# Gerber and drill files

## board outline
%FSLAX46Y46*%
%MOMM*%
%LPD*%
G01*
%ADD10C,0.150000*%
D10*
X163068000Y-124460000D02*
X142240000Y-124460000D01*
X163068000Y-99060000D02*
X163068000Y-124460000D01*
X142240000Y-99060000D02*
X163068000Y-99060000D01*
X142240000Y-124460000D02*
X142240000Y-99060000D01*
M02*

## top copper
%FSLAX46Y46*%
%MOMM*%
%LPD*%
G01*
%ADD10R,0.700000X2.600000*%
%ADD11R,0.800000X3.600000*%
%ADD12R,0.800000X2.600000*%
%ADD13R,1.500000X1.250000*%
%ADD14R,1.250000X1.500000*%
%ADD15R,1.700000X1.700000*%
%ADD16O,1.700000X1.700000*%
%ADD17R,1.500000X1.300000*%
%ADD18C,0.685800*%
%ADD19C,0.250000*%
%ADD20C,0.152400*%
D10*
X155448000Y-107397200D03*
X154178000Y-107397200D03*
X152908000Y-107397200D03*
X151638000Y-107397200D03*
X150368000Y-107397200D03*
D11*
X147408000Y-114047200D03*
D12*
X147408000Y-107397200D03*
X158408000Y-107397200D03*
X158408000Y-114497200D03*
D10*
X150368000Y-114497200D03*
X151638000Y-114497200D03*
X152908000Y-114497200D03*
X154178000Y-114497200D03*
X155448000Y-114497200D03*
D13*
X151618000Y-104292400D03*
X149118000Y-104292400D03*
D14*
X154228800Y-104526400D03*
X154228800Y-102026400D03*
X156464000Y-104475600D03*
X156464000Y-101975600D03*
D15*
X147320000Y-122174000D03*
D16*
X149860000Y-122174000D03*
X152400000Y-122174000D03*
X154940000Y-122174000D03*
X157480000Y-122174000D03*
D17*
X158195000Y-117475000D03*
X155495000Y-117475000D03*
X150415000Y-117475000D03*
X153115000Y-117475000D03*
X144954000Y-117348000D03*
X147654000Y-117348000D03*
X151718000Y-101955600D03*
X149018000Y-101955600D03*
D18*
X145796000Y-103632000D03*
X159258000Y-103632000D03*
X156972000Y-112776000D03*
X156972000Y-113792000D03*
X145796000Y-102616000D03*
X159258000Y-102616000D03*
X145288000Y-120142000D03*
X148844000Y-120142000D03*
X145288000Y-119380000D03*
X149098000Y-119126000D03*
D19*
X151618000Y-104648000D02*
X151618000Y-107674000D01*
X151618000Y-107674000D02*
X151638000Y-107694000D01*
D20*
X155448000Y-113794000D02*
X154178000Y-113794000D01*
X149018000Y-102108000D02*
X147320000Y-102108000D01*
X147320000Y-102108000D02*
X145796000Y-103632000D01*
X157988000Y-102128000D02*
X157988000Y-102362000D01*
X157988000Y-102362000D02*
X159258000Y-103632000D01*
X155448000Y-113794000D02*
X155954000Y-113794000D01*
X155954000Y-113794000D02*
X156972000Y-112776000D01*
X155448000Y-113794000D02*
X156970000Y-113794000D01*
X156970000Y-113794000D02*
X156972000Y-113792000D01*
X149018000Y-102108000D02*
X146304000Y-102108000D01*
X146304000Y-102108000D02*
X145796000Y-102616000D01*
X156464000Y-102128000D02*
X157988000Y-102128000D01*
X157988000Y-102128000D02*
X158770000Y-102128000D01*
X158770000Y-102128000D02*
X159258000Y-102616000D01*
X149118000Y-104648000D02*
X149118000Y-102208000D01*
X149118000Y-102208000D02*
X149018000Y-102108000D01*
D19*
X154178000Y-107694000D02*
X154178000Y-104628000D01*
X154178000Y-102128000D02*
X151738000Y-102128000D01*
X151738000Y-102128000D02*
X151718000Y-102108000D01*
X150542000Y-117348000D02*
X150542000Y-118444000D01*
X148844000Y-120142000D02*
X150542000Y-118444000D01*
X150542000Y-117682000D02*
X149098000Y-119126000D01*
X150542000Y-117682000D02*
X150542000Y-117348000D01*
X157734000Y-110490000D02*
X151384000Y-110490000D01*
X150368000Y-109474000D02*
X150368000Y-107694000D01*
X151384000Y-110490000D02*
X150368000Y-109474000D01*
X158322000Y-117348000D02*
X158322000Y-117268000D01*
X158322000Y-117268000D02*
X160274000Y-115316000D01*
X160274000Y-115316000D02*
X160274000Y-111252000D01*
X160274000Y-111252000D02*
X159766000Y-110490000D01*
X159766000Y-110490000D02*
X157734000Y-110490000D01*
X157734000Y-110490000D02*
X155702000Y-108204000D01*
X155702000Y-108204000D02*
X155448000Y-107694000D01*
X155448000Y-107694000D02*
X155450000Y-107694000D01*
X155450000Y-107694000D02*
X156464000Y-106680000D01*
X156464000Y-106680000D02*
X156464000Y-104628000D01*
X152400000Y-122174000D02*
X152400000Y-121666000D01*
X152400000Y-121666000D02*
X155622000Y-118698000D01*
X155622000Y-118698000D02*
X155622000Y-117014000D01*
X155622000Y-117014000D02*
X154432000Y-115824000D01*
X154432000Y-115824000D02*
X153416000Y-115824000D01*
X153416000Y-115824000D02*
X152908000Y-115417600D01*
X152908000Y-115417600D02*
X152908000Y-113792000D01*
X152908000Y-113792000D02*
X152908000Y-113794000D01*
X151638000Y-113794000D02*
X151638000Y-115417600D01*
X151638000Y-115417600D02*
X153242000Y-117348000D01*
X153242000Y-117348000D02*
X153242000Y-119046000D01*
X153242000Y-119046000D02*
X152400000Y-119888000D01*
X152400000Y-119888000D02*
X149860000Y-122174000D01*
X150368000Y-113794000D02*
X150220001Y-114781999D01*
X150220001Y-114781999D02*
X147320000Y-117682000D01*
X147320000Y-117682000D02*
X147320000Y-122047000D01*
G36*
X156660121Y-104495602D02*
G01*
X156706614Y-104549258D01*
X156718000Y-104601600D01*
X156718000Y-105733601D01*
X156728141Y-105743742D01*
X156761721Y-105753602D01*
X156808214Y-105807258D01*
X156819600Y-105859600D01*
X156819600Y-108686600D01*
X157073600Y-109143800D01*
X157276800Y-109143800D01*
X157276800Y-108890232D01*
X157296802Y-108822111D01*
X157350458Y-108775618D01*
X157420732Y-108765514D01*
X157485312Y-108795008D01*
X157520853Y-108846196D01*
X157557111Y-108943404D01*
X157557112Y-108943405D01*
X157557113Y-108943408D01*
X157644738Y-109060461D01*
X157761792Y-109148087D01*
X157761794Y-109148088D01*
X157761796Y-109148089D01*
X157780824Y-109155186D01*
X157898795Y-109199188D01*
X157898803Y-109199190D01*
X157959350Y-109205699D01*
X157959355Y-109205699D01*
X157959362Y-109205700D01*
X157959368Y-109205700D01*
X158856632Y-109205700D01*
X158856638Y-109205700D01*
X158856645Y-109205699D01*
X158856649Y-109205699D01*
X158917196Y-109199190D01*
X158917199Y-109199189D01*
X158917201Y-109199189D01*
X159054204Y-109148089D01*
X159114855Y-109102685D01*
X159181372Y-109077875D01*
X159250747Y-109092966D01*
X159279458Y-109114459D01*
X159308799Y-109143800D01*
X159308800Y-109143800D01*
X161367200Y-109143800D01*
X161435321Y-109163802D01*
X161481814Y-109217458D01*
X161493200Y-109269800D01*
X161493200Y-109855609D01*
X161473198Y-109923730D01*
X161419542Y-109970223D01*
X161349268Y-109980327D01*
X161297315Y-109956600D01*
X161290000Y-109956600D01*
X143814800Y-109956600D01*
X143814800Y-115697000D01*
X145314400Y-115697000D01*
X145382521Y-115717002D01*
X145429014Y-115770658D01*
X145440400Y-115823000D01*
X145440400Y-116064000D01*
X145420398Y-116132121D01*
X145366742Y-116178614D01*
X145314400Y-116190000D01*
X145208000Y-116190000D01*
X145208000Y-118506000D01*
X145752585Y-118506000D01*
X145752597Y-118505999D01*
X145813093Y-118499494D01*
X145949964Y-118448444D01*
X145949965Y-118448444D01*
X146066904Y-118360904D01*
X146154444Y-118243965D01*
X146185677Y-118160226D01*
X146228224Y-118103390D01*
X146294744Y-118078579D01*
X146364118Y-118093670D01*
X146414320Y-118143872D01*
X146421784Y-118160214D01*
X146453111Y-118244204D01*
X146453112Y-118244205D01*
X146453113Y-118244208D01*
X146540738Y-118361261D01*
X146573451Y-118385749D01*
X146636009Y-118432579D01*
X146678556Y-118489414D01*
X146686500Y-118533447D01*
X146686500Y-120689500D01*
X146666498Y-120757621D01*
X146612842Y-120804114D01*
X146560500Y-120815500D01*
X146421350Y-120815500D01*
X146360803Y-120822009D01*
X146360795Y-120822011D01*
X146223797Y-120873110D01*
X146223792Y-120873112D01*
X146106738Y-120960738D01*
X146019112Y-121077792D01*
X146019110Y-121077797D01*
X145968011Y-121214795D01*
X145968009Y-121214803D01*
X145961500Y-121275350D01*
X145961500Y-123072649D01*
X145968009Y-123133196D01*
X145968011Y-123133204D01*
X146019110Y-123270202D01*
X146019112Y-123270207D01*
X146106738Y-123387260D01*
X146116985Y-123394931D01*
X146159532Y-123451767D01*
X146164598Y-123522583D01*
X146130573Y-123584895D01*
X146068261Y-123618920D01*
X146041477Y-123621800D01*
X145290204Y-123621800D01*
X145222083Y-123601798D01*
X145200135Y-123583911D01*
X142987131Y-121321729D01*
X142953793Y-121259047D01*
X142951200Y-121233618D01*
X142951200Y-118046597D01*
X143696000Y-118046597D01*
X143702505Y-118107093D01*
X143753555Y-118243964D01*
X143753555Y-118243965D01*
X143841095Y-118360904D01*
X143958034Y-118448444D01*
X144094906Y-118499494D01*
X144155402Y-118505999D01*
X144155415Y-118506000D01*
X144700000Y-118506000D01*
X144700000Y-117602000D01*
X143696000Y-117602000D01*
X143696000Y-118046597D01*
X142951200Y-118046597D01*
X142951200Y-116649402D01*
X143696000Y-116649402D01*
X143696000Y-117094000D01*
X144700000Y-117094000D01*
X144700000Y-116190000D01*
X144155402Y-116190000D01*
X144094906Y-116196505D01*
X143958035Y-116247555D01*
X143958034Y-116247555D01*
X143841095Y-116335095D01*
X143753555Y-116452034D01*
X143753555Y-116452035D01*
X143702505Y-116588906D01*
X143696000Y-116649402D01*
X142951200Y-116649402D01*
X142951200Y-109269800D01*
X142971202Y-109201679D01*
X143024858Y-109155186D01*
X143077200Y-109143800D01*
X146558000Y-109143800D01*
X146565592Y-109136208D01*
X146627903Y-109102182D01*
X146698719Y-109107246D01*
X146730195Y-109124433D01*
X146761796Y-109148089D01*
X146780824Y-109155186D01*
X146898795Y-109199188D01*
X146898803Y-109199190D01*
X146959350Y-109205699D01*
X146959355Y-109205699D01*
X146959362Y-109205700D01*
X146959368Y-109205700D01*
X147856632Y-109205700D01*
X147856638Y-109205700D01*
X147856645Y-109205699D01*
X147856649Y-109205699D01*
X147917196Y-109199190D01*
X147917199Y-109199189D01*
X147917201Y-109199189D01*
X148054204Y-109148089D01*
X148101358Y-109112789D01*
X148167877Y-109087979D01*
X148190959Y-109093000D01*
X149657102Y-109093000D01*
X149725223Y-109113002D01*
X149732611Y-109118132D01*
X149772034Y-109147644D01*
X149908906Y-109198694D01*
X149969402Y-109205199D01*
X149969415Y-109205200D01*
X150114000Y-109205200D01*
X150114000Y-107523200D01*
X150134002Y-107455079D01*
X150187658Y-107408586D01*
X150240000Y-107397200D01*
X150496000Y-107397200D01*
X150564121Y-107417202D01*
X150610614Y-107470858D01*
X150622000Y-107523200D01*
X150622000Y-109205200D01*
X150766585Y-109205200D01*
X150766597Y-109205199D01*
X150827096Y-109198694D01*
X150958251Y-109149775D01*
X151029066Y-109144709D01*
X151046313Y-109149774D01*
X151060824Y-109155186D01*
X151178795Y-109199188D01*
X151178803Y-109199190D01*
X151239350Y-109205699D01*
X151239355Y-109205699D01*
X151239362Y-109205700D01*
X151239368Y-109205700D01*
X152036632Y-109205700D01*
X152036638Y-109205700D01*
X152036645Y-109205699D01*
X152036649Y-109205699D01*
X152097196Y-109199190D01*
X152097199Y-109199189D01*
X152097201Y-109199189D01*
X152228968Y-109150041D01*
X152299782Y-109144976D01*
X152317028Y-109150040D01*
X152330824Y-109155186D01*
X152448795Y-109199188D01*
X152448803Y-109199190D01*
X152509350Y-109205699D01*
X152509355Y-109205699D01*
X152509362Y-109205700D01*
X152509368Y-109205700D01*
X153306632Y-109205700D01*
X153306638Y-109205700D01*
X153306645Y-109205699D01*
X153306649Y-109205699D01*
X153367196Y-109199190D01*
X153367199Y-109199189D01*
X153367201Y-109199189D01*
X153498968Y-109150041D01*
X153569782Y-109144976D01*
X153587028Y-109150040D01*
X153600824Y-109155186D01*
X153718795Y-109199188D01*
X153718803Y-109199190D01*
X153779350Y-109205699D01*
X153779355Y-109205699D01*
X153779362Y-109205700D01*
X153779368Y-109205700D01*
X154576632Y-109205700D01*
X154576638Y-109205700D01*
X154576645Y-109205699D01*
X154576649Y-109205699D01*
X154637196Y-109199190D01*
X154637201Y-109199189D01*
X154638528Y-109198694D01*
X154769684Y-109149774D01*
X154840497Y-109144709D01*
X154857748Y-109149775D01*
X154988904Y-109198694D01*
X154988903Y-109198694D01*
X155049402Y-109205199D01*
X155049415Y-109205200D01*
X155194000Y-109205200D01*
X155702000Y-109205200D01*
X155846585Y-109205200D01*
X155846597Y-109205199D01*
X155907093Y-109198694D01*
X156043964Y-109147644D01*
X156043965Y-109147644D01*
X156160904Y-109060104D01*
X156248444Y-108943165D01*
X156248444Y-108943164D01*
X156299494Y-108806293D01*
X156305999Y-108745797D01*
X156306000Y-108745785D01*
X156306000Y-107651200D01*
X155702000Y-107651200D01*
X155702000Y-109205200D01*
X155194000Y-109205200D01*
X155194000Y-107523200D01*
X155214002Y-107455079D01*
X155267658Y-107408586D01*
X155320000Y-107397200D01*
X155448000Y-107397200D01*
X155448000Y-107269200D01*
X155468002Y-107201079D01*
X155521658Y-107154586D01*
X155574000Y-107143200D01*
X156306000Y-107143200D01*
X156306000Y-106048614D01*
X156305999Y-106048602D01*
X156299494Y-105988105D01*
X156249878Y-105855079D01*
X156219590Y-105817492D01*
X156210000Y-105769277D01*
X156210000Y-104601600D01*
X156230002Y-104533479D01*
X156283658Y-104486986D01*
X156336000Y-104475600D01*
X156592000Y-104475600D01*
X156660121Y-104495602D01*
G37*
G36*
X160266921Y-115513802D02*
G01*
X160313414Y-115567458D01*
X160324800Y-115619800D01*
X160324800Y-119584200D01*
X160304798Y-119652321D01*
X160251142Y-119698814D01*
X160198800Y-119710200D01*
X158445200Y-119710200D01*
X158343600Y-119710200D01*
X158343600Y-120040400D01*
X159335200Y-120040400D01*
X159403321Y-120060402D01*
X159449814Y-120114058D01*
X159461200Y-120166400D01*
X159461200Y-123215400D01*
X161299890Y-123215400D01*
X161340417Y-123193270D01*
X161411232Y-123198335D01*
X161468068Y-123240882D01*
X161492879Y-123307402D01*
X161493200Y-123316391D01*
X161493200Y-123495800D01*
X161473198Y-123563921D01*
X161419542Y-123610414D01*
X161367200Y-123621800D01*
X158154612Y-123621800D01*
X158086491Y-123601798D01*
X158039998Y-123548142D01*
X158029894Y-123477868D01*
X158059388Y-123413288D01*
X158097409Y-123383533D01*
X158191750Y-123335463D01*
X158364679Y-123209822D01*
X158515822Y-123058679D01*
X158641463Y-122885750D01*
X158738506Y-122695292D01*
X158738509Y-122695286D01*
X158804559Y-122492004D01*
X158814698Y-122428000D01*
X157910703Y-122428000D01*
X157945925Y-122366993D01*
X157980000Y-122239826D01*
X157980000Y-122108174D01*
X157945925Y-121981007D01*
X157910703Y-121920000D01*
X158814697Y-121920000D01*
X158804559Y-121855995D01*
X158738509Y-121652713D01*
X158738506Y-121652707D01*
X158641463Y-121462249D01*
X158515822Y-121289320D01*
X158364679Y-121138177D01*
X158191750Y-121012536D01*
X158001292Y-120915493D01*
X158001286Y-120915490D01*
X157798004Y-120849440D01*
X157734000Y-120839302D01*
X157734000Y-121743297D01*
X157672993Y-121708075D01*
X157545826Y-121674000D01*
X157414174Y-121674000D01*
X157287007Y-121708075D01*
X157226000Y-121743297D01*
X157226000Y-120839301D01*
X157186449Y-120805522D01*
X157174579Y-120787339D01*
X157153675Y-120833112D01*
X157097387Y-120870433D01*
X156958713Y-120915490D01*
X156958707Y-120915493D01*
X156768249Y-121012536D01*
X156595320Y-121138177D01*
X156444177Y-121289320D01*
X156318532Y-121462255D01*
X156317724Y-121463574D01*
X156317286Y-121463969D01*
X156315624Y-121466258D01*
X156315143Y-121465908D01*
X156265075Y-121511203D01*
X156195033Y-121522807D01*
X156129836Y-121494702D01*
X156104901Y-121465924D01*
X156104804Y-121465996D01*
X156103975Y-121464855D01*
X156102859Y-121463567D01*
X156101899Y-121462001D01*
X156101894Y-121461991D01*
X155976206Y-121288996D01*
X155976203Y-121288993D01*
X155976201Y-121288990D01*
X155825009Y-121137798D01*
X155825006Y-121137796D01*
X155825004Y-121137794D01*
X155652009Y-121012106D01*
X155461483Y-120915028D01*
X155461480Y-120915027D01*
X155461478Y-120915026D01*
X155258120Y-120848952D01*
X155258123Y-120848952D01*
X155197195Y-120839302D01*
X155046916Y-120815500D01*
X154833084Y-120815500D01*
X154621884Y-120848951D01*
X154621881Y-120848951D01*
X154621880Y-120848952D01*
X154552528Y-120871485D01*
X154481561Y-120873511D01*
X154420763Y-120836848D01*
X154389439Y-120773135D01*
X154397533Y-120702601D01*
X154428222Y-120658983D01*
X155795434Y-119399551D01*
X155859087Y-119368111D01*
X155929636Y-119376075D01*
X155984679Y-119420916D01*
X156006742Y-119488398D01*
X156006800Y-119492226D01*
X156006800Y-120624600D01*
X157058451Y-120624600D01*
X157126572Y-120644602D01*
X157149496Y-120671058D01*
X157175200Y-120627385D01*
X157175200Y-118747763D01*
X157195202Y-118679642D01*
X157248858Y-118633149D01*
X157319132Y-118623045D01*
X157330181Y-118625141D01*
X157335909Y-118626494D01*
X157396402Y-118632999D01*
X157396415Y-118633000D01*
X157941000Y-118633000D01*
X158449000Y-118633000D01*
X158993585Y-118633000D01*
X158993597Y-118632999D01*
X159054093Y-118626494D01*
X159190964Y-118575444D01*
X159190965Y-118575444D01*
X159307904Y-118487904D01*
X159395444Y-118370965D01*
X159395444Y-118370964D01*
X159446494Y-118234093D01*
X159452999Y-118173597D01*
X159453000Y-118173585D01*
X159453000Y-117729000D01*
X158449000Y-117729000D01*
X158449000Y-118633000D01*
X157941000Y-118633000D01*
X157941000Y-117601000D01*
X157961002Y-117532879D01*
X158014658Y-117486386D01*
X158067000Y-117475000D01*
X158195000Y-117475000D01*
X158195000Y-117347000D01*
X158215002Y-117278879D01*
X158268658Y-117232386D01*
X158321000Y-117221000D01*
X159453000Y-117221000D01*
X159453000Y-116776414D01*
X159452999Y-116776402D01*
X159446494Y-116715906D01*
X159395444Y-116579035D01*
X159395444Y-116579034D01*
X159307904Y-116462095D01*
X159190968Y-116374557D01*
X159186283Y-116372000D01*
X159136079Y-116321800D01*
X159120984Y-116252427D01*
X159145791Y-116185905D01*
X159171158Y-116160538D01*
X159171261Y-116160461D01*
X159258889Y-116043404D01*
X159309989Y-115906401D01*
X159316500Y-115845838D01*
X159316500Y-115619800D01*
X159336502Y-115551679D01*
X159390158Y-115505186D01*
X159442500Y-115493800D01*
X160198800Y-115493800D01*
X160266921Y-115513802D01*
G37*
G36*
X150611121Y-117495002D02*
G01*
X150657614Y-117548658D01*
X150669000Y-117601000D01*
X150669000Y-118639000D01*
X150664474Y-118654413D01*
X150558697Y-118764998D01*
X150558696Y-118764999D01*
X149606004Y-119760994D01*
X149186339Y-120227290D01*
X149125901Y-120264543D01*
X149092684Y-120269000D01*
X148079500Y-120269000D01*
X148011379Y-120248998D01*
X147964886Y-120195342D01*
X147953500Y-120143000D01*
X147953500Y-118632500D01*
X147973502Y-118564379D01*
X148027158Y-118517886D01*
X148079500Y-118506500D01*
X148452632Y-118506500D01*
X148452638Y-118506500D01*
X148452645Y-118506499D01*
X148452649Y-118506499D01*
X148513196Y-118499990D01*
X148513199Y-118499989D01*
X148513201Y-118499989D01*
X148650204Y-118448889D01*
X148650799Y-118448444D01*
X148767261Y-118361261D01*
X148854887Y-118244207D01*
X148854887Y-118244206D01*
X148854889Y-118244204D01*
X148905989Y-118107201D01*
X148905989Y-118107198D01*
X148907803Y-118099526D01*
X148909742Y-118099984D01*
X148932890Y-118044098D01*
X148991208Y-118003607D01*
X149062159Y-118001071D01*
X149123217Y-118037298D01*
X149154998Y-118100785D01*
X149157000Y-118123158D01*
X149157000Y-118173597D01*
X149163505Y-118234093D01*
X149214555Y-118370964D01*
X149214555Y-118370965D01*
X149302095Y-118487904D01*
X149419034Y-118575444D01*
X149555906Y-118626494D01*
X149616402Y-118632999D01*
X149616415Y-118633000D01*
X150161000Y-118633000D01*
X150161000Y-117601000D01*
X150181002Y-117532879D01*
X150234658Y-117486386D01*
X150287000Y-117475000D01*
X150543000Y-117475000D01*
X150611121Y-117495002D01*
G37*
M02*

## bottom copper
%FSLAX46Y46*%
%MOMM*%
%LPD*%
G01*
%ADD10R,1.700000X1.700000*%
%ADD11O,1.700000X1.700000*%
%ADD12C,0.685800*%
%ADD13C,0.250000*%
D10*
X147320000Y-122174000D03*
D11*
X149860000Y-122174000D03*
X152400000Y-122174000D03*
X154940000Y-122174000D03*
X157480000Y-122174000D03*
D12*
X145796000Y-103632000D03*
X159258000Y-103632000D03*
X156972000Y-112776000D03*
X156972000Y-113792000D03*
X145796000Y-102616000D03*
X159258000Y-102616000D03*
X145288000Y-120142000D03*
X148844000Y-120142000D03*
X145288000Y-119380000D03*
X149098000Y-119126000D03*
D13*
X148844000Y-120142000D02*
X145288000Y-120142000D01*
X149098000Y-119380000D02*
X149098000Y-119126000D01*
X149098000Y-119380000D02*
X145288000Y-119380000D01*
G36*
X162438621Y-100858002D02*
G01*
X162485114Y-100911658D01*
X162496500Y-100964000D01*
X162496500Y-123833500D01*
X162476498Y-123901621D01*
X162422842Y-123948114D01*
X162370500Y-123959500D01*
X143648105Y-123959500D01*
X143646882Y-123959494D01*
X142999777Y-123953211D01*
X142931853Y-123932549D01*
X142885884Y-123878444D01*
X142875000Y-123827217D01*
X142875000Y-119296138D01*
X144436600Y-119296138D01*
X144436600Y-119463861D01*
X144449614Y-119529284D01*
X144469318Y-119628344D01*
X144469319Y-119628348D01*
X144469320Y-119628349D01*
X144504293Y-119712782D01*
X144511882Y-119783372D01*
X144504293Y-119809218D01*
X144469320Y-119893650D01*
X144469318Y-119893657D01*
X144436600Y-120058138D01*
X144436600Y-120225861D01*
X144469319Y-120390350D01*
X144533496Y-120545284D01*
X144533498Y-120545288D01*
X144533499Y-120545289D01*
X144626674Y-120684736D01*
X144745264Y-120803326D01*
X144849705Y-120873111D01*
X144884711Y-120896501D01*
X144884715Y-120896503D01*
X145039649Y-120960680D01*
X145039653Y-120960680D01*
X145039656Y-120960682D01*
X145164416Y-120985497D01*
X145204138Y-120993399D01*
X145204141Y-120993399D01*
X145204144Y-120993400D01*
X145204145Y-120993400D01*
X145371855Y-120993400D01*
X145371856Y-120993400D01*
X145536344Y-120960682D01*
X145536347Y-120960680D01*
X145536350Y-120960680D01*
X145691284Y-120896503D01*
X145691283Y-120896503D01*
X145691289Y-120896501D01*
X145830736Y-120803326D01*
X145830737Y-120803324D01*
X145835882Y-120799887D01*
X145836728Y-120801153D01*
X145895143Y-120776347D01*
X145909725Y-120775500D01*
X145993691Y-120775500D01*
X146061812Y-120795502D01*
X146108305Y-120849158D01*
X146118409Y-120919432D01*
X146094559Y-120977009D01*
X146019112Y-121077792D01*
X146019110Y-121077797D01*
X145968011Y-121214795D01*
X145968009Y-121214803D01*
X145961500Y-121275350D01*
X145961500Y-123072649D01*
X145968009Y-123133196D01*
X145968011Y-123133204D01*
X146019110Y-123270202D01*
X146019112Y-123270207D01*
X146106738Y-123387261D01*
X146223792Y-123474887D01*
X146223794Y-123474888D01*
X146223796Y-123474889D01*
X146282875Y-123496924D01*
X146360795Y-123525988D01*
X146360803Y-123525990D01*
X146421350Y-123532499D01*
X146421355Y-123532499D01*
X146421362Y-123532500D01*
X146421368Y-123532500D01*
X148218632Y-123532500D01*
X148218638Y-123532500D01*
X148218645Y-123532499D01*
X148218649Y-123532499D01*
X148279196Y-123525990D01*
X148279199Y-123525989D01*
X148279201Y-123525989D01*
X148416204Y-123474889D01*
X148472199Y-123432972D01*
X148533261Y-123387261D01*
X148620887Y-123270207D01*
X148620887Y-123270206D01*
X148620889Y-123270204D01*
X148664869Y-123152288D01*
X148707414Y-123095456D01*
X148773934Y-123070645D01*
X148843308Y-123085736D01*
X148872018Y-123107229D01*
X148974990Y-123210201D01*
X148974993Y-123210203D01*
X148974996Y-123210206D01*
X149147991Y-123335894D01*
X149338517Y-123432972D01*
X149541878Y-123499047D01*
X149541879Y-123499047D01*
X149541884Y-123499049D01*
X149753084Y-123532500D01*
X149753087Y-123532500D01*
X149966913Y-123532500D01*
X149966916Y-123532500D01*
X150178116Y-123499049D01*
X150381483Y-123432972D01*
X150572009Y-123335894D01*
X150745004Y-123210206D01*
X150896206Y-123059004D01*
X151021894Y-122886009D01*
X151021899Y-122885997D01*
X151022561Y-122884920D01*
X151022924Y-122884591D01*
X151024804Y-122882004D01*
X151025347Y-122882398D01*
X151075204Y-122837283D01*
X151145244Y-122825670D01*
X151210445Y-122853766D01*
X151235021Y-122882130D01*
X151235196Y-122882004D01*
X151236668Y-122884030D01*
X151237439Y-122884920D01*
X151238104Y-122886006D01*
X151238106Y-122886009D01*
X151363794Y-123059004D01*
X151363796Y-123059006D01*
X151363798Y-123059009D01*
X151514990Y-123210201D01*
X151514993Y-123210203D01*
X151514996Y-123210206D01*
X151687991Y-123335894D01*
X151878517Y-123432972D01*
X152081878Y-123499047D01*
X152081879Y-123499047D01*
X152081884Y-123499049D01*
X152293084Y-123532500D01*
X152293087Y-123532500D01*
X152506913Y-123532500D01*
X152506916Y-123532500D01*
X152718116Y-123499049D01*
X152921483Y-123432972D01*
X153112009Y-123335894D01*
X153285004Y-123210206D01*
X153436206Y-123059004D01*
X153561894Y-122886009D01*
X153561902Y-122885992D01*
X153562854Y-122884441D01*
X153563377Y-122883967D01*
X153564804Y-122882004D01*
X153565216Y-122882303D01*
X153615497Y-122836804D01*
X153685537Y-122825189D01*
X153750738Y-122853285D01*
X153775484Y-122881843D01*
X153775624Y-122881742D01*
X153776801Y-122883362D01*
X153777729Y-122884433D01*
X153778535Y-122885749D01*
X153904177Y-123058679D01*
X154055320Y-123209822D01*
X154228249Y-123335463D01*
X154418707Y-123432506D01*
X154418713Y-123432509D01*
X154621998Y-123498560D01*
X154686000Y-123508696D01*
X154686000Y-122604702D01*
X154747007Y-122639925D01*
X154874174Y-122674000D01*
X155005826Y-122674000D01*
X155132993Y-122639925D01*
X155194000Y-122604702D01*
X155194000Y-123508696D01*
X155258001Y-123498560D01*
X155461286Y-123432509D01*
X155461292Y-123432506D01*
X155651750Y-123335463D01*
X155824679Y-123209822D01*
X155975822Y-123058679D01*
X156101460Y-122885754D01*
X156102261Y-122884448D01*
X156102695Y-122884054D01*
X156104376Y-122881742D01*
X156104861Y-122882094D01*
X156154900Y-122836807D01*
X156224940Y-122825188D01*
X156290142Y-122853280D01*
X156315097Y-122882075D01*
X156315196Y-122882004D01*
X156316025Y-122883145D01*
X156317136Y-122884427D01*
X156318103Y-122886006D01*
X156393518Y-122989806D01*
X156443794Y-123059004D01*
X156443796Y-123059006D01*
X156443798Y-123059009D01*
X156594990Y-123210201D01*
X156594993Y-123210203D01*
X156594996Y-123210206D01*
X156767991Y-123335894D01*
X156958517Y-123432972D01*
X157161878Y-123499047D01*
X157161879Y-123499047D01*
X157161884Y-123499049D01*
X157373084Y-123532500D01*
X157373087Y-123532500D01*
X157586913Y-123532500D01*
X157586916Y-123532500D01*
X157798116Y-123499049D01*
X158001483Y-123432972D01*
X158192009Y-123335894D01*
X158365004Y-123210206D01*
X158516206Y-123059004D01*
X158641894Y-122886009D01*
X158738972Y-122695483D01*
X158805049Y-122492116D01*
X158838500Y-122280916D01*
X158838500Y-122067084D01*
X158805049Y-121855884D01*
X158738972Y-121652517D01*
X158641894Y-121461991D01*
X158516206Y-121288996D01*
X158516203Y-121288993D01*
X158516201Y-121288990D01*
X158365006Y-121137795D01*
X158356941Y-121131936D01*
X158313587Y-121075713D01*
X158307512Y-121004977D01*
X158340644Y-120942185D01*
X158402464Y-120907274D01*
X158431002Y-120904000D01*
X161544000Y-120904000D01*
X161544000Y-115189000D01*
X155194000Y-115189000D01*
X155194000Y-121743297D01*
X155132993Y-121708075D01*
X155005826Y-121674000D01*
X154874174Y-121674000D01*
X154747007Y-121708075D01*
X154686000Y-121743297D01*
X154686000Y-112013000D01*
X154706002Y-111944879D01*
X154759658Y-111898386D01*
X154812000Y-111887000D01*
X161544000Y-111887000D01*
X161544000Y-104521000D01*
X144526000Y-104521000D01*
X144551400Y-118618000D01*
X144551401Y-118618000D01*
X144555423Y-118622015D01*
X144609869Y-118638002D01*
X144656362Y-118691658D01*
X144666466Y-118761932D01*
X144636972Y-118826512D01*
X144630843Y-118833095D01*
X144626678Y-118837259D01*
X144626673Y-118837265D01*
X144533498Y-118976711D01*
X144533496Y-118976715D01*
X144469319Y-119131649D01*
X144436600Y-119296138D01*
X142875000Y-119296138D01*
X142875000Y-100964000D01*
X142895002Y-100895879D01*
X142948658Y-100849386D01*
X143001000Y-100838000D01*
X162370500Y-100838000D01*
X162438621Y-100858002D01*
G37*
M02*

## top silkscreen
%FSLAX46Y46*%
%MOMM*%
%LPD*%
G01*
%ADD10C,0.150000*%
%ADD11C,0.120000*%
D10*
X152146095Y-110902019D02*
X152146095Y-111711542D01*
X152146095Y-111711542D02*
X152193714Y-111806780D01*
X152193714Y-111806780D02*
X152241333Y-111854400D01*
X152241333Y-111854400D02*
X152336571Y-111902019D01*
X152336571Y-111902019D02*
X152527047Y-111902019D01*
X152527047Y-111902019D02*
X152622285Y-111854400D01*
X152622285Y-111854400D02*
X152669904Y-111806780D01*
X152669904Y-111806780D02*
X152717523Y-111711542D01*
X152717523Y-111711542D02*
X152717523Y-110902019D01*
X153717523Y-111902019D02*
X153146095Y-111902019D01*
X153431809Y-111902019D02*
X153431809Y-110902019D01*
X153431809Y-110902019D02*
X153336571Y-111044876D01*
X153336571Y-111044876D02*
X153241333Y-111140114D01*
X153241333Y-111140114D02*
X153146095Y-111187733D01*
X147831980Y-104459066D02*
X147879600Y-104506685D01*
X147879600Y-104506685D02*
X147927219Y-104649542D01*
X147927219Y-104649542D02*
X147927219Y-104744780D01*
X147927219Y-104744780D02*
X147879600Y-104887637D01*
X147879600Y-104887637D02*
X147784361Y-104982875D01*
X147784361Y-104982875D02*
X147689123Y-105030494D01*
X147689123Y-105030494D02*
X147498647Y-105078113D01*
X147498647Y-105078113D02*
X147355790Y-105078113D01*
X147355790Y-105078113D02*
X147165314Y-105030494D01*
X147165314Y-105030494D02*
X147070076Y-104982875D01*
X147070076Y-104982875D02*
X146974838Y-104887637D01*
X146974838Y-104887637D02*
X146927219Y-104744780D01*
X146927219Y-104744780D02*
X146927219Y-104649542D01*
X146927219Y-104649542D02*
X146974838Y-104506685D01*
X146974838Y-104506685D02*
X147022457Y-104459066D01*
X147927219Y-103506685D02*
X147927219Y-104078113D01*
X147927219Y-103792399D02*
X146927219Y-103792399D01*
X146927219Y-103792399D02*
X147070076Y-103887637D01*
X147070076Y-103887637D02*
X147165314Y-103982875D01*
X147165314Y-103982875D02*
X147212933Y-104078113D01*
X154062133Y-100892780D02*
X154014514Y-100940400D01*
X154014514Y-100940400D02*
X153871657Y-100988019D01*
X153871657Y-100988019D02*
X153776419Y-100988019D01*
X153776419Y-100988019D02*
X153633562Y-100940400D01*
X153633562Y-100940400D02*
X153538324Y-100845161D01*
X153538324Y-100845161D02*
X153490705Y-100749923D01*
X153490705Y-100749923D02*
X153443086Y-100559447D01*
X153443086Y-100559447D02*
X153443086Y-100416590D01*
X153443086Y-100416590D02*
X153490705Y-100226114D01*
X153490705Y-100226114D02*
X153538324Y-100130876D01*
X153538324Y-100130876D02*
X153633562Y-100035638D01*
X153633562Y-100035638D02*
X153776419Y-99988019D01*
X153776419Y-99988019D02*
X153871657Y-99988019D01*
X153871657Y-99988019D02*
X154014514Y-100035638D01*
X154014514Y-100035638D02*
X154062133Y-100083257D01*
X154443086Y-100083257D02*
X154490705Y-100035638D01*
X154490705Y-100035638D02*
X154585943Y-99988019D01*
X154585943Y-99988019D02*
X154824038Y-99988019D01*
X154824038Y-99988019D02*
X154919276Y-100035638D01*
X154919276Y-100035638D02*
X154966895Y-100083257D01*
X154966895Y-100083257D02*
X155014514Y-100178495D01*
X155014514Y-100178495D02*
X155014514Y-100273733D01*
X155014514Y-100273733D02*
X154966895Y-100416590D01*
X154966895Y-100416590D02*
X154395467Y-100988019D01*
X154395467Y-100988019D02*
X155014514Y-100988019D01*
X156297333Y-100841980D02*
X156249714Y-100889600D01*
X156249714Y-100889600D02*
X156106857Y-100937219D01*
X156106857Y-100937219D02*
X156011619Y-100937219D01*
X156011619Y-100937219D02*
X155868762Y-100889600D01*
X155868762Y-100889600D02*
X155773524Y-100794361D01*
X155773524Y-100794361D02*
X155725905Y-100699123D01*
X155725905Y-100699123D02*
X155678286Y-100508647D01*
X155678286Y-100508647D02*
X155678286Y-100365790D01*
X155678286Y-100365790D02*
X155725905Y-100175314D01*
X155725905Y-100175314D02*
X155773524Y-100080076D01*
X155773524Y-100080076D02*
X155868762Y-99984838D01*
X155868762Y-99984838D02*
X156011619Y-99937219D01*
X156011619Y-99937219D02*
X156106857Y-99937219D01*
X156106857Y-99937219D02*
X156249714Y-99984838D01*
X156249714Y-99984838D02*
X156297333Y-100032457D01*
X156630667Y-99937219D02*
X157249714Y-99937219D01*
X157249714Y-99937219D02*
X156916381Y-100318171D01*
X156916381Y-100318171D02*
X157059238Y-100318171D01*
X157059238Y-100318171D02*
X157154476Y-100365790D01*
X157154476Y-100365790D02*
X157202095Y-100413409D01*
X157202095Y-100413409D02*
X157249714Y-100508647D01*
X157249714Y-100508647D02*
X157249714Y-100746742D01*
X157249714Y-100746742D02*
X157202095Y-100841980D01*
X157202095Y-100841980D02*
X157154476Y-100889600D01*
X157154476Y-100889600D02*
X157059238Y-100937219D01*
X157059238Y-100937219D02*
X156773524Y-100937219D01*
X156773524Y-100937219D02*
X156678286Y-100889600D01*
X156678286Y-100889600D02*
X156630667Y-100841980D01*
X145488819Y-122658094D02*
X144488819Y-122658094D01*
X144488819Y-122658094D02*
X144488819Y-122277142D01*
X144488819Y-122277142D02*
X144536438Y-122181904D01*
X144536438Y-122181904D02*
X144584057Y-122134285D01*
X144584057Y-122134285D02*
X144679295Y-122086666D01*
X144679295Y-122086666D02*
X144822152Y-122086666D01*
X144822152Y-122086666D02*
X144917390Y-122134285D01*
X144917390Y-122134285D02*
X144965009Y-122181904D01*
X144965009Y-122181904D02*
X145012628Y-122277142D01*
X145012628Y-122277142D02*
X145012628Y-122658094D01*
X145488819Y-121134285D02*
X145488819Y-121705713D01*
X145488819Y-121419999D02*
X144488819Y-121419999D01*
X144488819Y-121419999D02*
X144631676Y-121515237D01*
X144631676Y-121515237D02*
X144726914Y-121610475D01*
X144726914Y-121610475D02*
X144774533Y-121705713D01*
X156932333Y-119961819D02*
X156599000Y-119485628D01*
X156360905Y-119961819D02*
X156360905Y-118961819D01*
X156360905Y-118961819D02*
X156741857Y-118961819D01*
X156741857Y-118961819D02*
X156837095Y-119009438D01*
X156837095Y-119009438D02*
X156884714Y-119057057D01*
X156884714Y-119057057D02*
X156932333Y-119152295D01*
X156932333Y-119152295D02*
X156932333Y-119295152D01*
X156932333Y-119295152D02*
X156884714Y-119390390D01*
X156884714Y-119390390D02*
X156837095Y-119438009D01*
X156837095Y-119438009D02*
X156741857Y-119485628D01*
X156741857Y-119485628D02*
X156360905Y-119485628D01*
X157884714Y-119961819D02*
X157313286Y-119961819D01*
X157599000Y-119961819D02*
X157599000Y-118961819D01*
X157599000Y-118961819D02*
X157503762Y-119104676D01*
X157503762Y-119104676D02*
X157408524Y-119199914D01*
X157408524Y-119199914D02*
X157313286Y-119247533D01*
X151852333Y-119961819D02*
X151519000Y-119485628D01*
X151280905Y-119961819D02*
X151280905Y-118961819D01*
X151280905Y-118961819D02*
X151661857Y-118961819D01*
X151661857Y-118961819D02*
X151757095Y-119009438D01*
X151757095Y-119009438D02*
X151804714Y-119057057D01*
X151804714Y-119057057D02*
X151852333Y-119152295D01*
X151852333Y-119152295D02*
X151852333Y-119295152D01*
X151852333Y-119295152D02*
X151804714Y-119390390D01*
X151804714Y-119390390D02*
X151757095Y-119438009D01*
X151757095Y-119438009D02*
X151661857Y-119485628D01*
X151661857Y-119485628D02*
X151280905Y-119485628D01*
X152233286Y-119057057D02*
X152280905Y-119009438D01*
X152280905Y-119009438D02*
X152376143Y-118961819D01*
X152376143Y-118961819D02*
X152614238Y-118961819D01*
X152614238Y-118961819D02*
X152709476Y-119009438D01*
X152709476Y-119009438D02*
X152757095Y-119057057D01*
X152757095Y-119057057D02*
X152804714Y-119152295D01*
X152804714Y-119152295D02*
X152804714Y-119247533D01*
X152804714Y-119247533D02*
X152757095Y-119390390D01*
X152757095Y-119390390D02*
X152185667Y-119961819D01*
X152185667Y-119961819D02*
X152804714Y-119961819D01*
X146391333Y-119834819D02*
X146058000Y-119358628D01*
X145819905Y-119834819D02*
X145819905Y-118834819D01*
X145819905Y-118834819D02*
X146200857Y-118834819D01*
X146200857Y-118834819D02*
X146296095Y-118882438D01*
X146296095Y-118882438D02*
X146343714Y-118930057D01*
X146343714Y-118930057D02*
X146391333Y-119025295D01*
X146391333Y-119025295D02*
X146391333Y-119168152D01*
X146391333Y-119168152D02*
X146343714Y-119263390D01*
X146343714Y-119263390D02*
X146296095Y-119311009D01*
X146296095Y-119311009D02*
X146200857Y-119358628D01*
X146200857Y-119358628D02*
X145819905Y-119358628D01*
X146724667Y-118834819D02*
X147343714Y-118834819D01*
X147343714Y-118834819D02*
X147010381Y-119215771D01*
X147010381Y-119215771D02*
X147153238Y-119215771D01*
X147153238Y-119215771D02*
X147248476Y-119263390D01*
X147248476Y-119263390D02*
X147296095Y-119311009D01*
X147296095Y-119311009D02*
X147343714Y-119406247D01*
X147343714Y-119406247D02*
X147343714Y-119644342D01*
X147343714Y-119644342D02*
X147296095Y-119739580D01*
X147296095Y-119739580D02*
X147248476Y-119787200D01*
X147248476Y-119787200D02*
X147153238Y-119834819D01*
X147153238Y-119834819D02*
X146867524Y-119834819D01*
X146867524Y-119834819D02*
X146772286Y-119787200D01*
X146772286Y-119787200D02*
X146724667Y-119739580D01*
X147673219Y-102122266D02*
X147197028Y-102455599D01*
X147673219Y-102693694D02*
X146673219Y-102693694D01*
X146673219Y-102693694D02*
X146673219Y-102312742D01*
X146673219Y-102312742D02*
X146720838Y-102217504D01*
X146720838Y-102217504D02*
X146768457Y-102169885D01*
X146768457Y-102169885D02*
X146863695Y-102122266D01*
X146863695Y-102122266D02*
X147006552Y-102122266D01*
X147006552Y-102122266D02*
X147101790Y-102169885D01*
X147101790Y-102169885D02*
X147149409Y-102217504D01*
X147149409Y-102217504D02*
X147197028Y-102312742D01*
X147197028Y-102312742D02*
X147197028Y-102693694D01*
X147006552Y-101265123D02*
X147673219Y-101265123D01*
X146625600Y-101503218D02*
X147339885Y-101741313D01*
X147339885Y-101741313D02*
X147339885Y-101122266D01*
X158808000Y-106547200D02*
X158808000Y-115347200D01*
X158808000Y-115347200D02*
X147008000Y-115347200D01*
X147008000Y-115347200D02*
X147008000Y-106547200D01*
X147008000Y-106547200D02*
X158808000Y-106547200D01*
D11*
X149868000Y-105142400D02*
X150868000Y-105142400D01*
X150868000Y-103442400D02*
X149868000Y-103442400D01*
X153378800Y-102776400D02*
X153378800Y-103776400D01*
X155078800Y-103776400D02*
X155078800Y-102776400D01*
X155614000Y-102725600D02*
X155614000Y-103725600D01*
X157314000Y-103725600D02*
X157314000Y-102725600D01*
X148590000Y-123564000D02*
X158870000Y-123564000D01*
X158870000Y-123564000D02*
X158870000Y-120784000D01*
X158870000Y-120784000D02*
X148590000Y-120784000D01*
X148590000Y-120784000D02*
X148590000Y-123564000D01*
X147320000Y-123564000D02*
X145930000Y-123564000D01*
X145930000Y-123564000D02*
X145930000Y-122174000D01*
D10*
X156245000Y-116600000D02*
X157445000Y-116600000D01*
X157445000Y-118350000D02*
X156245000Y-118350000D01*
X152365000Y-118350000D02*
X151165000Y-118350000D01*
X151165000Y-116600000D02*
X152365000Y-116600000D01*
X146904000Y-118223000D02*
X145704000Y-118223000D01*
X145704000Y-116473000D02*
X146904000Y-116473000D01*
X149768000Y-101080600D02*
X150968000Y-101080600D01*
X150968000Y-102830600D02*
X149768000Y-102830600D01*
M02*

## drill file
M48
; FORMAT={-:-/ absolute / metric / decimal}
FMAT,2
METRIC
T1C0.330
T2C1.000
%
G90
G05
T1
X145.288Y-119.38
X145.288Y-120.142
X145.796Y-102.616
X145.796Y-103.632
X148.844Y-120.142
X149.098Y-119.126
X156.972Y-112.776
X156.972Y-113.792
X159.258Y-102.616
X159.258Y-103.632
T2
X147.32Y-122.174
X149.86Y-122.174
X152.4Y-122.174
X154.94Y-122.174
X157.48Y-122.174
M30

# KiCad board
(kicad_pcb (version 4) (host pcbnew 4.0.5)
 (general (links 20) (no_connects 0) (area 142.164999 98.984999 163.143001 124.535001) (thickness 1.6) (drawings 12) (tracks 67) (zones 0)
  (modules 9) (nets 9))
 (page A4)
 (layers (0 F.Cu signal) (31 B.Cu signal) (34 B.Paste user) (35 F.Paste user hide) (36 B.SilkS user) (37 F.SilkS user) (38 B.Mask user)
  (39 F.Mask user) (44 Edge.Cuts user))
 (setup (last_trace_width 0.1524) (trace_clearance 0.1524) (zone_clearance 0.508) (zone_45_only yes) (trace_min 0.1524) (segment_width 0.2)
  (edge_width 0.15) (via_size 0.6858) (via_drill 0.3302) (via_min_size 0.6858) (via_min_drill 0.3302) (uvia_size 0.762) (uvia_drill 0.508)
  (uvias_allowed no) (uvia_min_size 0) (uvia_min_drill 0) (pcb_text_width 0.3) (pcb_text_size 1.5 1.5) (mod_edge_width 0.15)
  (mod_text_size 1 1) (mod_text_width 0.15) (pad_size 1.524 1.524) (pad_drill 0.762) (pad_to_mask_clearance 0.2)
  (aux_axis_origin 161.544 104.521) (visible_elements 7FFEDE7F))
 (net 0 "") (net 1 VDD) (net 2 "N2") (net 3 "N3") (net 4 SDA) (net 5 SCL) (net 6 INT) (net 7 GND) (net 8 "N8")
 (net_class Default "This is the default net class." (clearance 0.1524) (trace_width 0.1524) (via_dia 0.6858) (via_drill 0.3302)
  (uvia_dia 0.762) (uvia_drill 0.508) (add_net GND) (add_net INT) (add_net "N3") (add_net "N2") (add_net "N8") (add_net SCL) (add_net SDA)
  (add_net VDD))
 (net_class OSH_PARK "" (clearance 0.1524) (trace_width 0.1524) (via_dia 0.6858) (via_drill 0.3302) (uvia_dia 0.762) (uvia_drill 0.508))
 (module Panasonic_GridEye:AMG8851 (layer F.Cu) (at 152.908 110.9472)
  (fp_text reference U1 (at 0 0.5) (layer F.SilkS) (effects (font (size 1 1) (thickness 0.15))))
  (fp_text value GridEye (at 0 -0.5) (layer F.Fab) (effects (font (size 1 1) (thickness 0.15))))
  (fp_line (start 5.9 -4.4) (end 5.9 4.4) (layer F.SilkS) (width 0.15))
  (fp_line (start 5.9 4.4) (end -5.9 4.4) (layer F.SilkS) (width 0.15))
  (fp_line (start -5.9 4.4) (end -5.9 -4.4) (layer F.SilkS) (width 0.15))
  (fp_line (start -5.9 -4.4) (end 5.9 -4.4) (layer F.SilkS) (width 0.15))
  (pad 9 smd rect (at 2.54 -3.55) (size 0.7 2.6) (layers F.Cu F.Paste F.Mask) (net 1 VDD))
  (pad 10 smd rect (at 1.27 -3.55) (size 0.7 2.6) (layers F.Cu F.Paste F.Mask) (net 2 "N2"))
  (pad 11 smd rect (at 0 -3.55) (size 0.7 2.6) (layers F.Cu F.Paste F.Mask))
  (pad 12 smd rect (at -1.27 -3.55) (size 0.7 2.6) (layers F.Cu F.Paste F.Mask) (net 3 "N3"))
  (pad 13 smd rect (at -2.54 -3.55) (size 0.7 2.6) (layers F.Cu F.Paste F.Mask) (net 1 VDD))
  (pad 1 smd rect (at -5.5 3.1) (size 0.8 3.6) (layers F.Cu F.Paste F.Mask))
  (pad 14 smd rect (at -5.5 -3.55) (size 0.8 2.6) (layers F.Cu F.Paste F.Mask))
  (pad 8 smd rect (at 5.5 -3.55) (size 0.8 2.6) (layers F.Cu F.Paste F.Mask))
  (pad 7 smd rect (at 5.5 3.55) (size 0.8 2.6) (layers F.Cu F.Paste F.Mask))
  (pad 2 smd rect (at -2.54 3.55) (size 0.7 2.6) (layers F.Cu F.Paste F.Mask) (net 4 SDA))
  (pad 3 smd rect (at -1.27 3.55) (size 0.7 2.6) (layers F.Cu F.Paste F.Mask) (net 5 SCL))
  (pad 4 smd rect (at 0 3.55) (size 0.7 2.6) (layers F.Cu F.Paste F.Mask) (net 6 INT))
  (pad 5 smd rect (at 1.27 3.55) (size 0.7 2.6) (layers F.Cu F.Paste F.Mask) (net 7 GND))
  (pad 6 smd rect (at 2.54 3.55) (size 0.7 2.6) (layers F.Cu F.Paste F.Mask) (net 7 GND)))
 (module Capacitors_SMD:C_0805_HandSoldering (layer F.Cu) (at 150.368 104.2924 180)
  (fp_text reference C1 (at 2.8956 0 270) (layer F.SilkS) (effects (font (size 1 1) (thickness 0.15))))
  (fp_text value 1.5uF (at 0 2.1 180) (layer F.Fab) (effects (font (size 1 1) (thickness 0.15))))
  (fp_line (start 0.5 -0.85) (end -0.5 -0.85) (layer F.SilkS) (width 0.12))
  (fp_line (start -0.5 0.85) (end 0.5 0.85) (layer F.SilkS) (width 0.12))
  (pad 1 smd rect (at -1.25 0 180) (size 1.5 1.25) (layers F.Cu F.Paste F.Mask) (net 3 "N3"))
  (pad 2 smd rect (at 1.25 0 180) (size 1.5 1.25) (layers F.Cu F.Paste F.Mask) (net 7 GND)))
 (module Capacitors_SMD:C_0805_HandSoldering (layer F.Cu) (at 154.2288 103.2764 90)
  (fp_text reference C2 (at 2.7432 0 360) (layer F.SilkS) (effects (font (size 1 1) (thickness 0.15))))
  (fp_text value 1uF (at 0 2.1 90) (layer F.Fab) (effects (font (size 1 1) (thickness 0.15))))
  (fp_line (start 0.5 -0.85) (end -0.5 -0.85) (layer F.SilkS) (width 0.12))
  (fp_line (start -0.5 0.85) (end 0.5 0.85) (layer F.SilkS) (width 0.12))
  (pad 1 smd rect (at -1.25 0 90) (size 1.5 1.25) (layers F.Cu F.Paste F.Mask) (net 2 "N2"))
  (pad 2 smd rect (at 1.25 0 90) (size 1.5 1.25) (layers F.Cu F.Paste F.Mask) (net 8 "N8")))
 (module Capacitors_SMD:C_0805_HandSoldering (layer F.Cu) (at 156.464 103.2256 90)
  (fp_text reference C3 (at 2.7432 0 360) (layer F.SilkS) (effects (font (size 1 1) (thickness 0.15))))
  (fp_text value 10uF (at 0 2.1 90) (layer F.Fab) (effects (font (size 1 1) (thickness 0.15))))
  (fp_line (start 0.5 -0.85) (end -0.5 -0.85) (layer F.SilkS) (width 0.12))
  (fp_line (start -0.5 0.85) (end 0.5 0.85) (layer F.SilkS) (width 0.12))
  (pad 1 smd rect (at -1.25 0 90) (size 1.5 1.25) (layers F.Cu F.Paste F.Mask) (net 1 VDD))
  (pad 2 smd rect (at 1.25 0 90) (size 1.5 1.25) (layers F.Cu F.Paste F.Mask) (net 7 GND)))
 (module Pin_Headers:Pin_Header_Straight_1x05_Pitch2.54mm (layer F.Cu) (at 147.32 122.174 90)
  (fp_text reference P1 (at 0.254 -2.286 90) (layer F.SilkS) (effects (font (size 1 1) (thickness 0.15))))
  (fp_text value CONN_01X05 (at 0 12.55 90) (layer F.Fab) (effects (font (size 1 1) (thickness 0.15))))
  (fp_line (start -1.39 1.27) (end -1.39 11.55) (layer F.SilkS) (width 0.12))
  (fp_line (start -1.39 11.55) (end 1.39 11.55) (layer F.SilkS) (width 0.12))
  (fp_line (start 1.39 11.55) (end 1.39 1.27) (layer F.SilkS) (width 0.12))
  (fp_line (start 1.39 1.27) (end -1.39 1.27) (layer F.SilkS) (width 0.12))
  (fp_line (start -1.39 0) (end -1.39 -1.39) (layer F.SilkS) (width 0.12))
  (fp_line (start -1.39 -1.39) (end 0 -1.39) (layer F.SilkS) (width 0.12))
  (pad 1 thru_hole rect (at 0 0 90) (size 1.7 1.7) (drill 1) (layers *.Cu *.Mask) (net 4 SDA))
  (pad 2 thru_hole oval (at 0 2.54 90) (size 1.7 1.7) (drill 1) (layers *.Cu *.Mask) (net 5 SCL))
  (pad 3 thru_hole oval (at 0 5.08 90) (size 1.7 1.7) (drill 1) (layers *.Cu *.Mask) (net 6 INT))
  (pad 4 thru_hole oval (at 0 7.62 90) (size 1.7 1.7) (drill 1) (layers *.Cu *.Mask) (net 7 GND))
  (pad 5 thru_hole oval (at 0 10.16 90) (size 1.7 1.7) (drill 1) (layers *.Cu *.Mask) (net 1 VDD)))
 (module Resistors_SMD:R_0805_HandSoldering (layer F.Cu) (at 156.845 117.475 180)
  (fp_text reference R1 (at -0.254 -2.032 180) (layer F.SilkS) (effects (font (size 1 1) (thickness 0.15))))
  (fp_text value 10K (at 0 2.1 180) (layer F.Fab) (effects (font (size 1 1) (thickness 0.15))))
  (fp_line (start 0.6 0.875) (end -0.6 0.875) (layer F.SilkS) (width 0.15))
  (fp_line (start -0.6 -0.875) (end 0.6 -0.875) (layer F.SilkS) (width 0.15))
  (pad 1 smd rect (at -1.35 0 180) (size 1.5 1.3) (layers F.Cu F.Paste F.Mask) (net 1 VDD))
  (pad 2 smd rect (at 1.35 0 180) (size 1.5 1.3) (layers F.Cu F.Paste F.Mask) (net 6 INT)))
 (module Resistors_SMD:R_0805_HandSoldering (layer F.Cu) (at 151.765 117.475)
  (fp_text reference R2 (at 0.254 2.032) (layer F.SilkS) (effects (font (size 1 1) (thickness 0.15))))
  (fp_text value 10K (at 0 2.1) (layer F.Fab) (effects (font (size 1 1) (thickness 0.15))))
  (fp_line (start 0.6 0.875) (end -0.6 0.875) (layer F.SilkS) (width 0.15))
  (fp_line (start -0.6 -0.875) (end 0.6 -0.875) (layer F.SilkS) (width 0.15))
  (pad 1 smd rect (at -1.35 0) (size 1.5 1.3) (layers F.Cu F.Paste F.Mask) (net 1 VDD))
  (pad 2 smd rect (at 1.35 0) (size 1.5 1.3) (layers F.Cu F.Paste F.Mask) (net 5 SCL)))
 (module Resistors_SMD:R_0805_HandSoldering (layer F.Cu) (at 146.304 117.348)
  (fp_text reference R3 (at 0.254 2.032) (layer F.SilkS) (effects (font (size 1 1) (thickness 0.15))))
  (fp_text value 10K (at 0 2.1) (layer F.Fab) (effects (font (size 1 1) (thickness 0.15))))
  (fp_line (start 0.6 0.875) (end -0.6 0.875) (layer F.SilkS) (width 0.15))
  (fp_line (start -0.6 -0.875) (end 0.6 -0.875) (layer F.SilkS) (width 0.15))
  (pad 1 smd rect (at -1.35 0) (size 1.5 1.3) (layers F.Cu F.Paste F.Mask) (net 1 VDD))
  (pad 2 smd rect (at 1.35 0) (size 1.5 1.3) (layers F.Cu F.Paste F.Mask) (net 4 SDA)))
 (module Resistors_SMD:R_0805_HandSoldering (layer F.Cu) (at 150.368 101.9556 180)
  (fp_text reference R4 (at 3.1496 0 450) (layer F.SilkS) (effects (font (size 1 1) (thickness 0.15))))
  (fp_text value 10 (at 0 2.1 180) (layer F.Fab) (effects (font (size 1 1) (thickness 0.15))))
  (fp_line (start 0.6 0.875) (end -0.6 0.875) (layer F.SilkS) (width 0.15))
  (fp_line (start -0.6 -0.875) (end 0.6 -0.875) (layer F.SilkS) (width 0.15))
  (pad 1 smd rect (at -1.35 0 180) (size 1.5 1.3) (layers F.Cu F.Paste F.Mask) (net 8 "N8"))
  (pad 2 smd rect (at 1.35 0 180) (size 1.5 1.3) (layers F.Cu F.Paste F.Mask) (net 7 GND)))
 (gr_line (start 163.068 124.46) (end 142.24 124.46) (angle 90) (layer Edge.Cuts) (width 0.15))
 (gr_line (start 163.068 99.06) (end 163.068 124.46) (angle 90) (layer Edge.Cuts) (width 0.15))
 (gr_line (start 142.24 99.06) (end 163.068 99.06) (angle 90) (layer Edge.Cuts) (width 0.15))
 (gr_line (start 142.24 124.46) (end 142.24 99.06) (angle 90) (layer Edge.Cuts) (width 0.15))
 (segment (start 151.618 104.648) (end 151.618 107.674) (width 0.25) (layer F.Cu) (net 3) (status 20))
 (segment (start 151.618 107.674) (end 151.638 107.694) (width 0.25) (layer F.Cu) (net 3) (status 30))
 (segment (start 155.448 113.794) (end 154.178 113.794) (width 0.1524) (layer F.Cu) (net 7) (status 30))
 (via (at 145.796 103.632) (size 0.6858) (drill 0.3302) (layers F.Cu B.Cu) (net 7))
 (segment (start 149.018 102.108) (end 147.32 102.108) (width 0.1524) (layer F.Cu) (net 7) (status 10))
 (segment (start 147.32 102.108) (end 145.796 103.632) (width 0.1524) (layer F.Cu) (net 7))
 (via (at 159.258 103.632) (size 0.6858) (drill 0.3302) (layers F.Cu B.Cu) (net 7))
 (segment (start 157.988 102.128) (end 157.988 102.362) (width 0.1524) (layer F.Cu) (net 7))
 (segment (start 157.988 102.362) (end 159.258 103.632) (width 0.1524) (layer F.Cu) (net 7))
 (via (at 156.972 112.776) (size 0.6858) (drill 0.3302) (layers F.Cu B.Cu) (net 7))
 (segment (start 155.448 113.794) (end 155.954 113.794) (width 0.1524) (layer F.Cu) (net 7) (status 10))
 (segment (start 155.954 113.794) (end 156.972 112.776) (width 0.1524) (layer F.Cu) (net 7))
 (via (at 156.972 113.792) (size 0.6858) (drill 0.3302) (layers F.Cu B.Cu) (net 7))
 (segment (start 155.448 113.794) (end 156.97 113.794) (width 0.1524) (layer F.Cu) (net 7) (status 10))
 (segment (start 156.97 113.794) (end 156.972 113.792) (width 0.1524) (layer F.Cu) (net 7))
 (via (at 145.796 102.616) (size 0.6858) (drill 0.3302) (layers F.Cu B.Cu) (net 7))
 (segment (start 149.018 102.108) (end 146.304 102.108) (width 0.1524) (layer F.Cu) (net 7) (status 10))
 (segment (start 146.304 102.108) (end 145.796 102.616) (width 0.1524) (layer F.Cu) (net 7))
 (via (at 159.258 102.616) (size 0.6858) (drill 0.3302) (layers F.Cu B.Cu) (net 7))
 (segment (start 156.464 102.128) (end 157.988 102.128) (width 0.1524) (layer F.Cu) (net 7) (status 10))
 (segment (start 157.988 102.128) (end 158.77 102.128) (width 0.1524) (layer F.Cu) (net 7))
 (segment (start 158.77 102.128) (end 159.258 102.616) (width 0.1524) (layer F.Cu) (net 7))
 (segment (start 149.118 104.648) (end 149.118 102.208) (width 0.1524) (layer F.Cu) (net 7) (status 30))
 (segment (start 149.118 102.208) (end 149.018 102.108) (width 0.1524) (layer F.Cu) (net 7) (status 30))
 (segment (start 154.178 107.694) (end 154.178 104.628) (width 0.25) (layer F.Cu) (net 2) (status 10))
 (segment (start 154.178 102.128) (end 151.738 102.128) (width 0.25) (layer F.Cu) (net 8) (status 30))
 (segment (start 151.738 102.128) (end 151.718 102.108) (width 0.25) (layer F.Cu) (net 8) (status 30))
 (via (at 145.288 120.142) (size 0.6858) (drill 0.3302) (layers F.Cu B.Cu) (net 1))
 (segment (start 150.542 117.348) (end 150.542 118.444) (width 0.25) (layer F.Cu) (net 1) (status 10))
 (segment (start 148.844 120.142) (end 150.542 118.444) (width 0.25) (layer F.Cu) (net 1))
 (via (at 148.844 120.142) (size 0.6858) (drill 0.3302) (layers F.Cu B.Cu) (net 1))
 (segment (start 148.844 120.142) (end 145.288 120.142) (width 0.25) (layer B.Cu) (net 1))
 (via (at 145.288 119.38) (size 0.6858) (drill 0.3302) (layers F.Cu B.Cu) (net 1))
 (segment (start 150.542 117.682) (end 149.098 119.126) (width 0.25) (layer F.Cu) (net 1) (status 10))
 (via (at 149.098 119.126) (size 0.6858) (drill 0.3302) (layers F.Cu B.Cu) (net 1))
 (segment (start 149.098 119.38) (end 149.098 119.126) (width 0.25) (layer B.Cu) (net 1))
 (segment (start 149.098 119.38) (end 145.288 119.38) (width 0.25) (layer B.Cu) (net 1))
 (segment (start 150.542 117.682) (end 150.542 117.348) (width 0.25) (layer F.Cu) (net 1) (status 30))
 (segment (start 157.734 110.49) (end 151.384 110.49) (width 0.25) (layer F.Cu) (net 1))
 (segment (start 150.368 109.474) (end 150.368 107.694) (width 0.25) (layer F.Cu) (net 1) (status 20))
 (segment (start 151.384 110.49) (end 150.368 109.474) (width 0.25) (layer F.Cu) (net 1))
 (segment (start 158.322 117.348) (end 158.322 117.268) (width 0.25) (layer F.Cu) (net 1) (status 30))
 (segment (start 158.322 117.268) (end 160.274 115.316) (width 0.25) (layer F.Cu) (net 1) (status 10))
 (segment (start 160.274 115.316) (end 160.274 111.252) (width 0.25) (layer F.Cu) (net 1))
 (segment (start 160.274 111.252) (end 159.766 110.49) (width 0.25) (layer F.Cu) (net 1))
 (segment (start 159.766 110.49) (end 157.734 110.49) (width 0.25) (layer F.Cu) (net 1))
 (segment (start 157.734 110.49) (end 155.702 108.204) (width 0.25) (layer F.Cu) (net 1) (status 20))
 (segment (start 155.702 108.204) (end 155.448 107.694) (width 0.25) (layer F.Cu) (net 1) (status 30))
 (segment (start 155.448 107.694) (end 155.45 107.694) (width 0.25) (layer F.Cu) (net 1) (status 30))
 (segment (start 155.45 107.694) (end 156.464 106.68) (width 0.25) (layer F.Cu) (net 1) (status 10))
 (segment (start 156.464 106.68) (end 156.464 104.628) (width 0.25) (layer F.Cu) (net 1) (status 20))
 (segment (start 152.4 122.174) (end 152.4 121.666) (width 0.25) (layer F.Cu) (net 6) (status 30))
 (segment (start 152.4 121.666) (end 155.622 118.698) (width 0.25) (layer F.Cu) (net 6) (status 10))
 (segment (start 155.622 118.698) (end 155.622 117.014) (width 0.25) (layer F.Cu) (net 6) (status 20))
 (segment (start 155.622 117.014) (end 154.432 115.824) (width 0.25) (layer F.Cu) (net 6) (status 10))
 (segment (start 154.432 115.824) (end 153.416 115.824) (width 0.25) (layer F.Cu) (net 6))
 (segment (start 153.416 115.824) (end 152.908 115.4176) (width 0.25) (layer F.Cu) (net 6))
 (segment (start 152.908 115.4176) (end 152.908 113.792) (width 0.25) (layer F.Cu) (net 6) (status 20))
 (segment (start 152.908 113.792) (end 152.908 113.794) (width 0.25) (layer F.Cu) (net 6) (status 30))
 (segment (start 151.638 113.794) (end 151.638 115.4176) (width 0.25) (layer F.Cu) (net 5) (status 10))
 (segment (start 151.638 115.4176) (end 153.242 117.348) (width 0.25) (layer F.Cu) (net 5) (status 20))
 (segment (start 153.242 117.348) (end 153.242 119.046) (width 0.25) (layer F.Cu) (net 5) (status 10))
 (segment (start 153.242 119.046) (end 152.4 119.888) (width 0.25) (layer F.Cu) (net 5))
 (segment (start 152.4 119.888) (end 149.86 122.174) (width 0.25) (layer F.Cu) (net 5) (status 20))
 (segment (start 150.368 113.794) (end 150.220001 114.781999) (width 0.25) (layer F.Cu) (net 4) (status 30))
 (segment (start 150.220001 114.781999) (end 147.32 117.682) (width 0.25) (layer F.Cu) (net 4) (status 10))
 (segment (start 147.32 117.682) (end 147.32 122.047) (width 0.25) (layer F.Cu) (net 4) (status 30))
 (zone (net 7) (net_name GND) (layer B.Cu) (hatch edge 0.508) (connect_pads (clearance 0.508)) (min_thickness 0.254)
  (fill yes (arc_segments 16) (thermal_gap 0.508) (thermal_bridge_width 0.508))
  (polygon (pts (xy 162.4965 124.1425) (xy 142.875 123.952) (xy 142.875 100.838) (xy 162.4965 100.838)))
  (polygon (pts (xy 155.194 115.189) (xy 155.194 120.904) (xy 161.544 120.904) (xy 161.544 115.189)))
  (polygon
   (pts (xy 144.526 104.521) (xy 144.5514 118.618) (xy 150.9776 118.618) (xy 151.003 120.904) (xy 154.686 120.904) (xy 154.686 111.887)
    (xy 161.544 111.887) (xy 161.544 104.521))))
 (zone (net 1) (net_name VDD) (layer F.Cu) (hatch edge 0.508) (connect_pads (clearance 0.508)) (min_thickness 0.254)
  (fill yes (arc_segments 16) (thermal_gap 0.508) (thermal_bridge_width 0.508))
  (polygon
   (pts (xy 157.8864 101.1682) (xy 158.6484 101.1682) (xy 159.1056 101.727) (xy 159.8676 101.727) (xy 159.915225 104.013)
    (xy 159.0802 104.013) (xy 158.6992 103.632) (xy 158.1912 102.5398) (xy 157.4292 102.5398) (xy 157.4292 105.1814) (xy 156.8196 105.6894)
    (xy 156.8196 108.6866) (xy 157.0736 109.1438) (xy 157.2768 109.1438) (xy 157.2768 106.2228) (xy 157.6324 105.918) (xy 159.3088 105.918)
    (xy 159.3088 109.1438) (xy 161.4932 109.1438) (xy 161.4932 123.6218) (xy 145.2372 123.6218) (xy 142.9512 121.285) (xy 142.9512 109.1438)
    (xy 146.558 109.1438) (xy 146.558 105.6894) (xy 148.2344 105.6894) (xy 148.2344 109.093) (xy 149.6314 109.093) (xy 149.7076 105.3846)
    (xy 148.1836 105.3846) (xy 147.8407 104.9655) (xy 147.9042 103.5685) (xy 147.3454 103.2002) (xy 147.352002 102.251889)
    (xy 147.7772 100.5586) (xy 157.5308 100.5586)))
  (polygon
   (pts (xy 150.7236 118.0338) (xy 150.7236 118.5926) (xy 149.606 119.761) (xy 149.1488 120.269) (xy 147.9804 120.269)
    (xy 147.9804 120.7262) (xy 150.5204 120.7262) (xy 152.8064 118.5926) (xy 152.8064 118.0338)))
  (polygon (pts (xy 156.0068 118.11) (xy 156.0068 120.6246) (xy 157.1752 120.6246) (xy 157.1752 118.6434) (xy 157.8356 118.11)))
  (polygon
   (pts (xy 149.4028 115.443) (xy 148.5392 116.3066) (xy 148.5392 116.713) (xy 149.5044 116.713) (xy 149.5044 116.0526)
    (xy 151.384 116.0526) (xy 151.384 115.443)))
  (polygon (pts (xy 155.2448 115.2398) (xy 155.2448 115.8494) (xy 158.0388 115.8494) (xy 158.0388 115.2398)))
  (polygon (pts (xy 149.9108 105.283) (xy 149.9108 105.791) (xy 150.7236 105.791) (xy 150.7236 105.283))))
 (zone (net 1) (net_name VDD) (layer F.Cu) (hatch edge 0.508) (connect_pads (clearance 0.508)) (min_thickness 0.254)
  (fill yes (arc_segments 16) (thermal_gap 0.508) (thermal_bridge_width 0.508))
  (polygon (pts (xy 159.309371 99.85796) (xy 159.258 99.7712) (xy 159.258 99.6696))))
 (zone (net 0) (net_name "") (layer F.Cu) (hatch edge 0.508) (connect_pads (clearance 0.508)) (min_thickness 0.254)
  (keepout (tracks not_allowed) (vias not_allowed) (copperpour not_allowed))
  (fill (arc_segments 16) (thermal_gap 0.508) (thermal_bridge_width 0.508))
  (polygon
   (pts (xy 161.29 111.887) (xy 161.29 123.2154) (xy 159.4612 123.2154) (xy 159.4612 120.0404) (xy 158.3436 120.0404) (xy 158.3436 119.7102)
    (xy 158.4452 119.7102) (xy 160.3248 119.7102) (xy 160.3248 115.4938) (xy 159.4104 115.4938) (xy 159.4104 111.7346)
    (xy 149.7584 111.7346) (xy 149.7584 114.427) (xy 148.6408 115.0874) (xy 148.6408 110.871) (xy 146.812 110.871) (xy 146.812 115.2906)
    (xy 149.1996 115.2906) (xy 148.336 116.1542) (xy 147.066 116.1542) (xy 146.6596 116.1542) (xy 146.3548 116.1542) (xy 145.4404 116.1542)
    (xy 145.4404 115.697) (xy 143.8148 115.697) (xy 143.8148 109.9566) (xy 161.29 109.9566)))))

